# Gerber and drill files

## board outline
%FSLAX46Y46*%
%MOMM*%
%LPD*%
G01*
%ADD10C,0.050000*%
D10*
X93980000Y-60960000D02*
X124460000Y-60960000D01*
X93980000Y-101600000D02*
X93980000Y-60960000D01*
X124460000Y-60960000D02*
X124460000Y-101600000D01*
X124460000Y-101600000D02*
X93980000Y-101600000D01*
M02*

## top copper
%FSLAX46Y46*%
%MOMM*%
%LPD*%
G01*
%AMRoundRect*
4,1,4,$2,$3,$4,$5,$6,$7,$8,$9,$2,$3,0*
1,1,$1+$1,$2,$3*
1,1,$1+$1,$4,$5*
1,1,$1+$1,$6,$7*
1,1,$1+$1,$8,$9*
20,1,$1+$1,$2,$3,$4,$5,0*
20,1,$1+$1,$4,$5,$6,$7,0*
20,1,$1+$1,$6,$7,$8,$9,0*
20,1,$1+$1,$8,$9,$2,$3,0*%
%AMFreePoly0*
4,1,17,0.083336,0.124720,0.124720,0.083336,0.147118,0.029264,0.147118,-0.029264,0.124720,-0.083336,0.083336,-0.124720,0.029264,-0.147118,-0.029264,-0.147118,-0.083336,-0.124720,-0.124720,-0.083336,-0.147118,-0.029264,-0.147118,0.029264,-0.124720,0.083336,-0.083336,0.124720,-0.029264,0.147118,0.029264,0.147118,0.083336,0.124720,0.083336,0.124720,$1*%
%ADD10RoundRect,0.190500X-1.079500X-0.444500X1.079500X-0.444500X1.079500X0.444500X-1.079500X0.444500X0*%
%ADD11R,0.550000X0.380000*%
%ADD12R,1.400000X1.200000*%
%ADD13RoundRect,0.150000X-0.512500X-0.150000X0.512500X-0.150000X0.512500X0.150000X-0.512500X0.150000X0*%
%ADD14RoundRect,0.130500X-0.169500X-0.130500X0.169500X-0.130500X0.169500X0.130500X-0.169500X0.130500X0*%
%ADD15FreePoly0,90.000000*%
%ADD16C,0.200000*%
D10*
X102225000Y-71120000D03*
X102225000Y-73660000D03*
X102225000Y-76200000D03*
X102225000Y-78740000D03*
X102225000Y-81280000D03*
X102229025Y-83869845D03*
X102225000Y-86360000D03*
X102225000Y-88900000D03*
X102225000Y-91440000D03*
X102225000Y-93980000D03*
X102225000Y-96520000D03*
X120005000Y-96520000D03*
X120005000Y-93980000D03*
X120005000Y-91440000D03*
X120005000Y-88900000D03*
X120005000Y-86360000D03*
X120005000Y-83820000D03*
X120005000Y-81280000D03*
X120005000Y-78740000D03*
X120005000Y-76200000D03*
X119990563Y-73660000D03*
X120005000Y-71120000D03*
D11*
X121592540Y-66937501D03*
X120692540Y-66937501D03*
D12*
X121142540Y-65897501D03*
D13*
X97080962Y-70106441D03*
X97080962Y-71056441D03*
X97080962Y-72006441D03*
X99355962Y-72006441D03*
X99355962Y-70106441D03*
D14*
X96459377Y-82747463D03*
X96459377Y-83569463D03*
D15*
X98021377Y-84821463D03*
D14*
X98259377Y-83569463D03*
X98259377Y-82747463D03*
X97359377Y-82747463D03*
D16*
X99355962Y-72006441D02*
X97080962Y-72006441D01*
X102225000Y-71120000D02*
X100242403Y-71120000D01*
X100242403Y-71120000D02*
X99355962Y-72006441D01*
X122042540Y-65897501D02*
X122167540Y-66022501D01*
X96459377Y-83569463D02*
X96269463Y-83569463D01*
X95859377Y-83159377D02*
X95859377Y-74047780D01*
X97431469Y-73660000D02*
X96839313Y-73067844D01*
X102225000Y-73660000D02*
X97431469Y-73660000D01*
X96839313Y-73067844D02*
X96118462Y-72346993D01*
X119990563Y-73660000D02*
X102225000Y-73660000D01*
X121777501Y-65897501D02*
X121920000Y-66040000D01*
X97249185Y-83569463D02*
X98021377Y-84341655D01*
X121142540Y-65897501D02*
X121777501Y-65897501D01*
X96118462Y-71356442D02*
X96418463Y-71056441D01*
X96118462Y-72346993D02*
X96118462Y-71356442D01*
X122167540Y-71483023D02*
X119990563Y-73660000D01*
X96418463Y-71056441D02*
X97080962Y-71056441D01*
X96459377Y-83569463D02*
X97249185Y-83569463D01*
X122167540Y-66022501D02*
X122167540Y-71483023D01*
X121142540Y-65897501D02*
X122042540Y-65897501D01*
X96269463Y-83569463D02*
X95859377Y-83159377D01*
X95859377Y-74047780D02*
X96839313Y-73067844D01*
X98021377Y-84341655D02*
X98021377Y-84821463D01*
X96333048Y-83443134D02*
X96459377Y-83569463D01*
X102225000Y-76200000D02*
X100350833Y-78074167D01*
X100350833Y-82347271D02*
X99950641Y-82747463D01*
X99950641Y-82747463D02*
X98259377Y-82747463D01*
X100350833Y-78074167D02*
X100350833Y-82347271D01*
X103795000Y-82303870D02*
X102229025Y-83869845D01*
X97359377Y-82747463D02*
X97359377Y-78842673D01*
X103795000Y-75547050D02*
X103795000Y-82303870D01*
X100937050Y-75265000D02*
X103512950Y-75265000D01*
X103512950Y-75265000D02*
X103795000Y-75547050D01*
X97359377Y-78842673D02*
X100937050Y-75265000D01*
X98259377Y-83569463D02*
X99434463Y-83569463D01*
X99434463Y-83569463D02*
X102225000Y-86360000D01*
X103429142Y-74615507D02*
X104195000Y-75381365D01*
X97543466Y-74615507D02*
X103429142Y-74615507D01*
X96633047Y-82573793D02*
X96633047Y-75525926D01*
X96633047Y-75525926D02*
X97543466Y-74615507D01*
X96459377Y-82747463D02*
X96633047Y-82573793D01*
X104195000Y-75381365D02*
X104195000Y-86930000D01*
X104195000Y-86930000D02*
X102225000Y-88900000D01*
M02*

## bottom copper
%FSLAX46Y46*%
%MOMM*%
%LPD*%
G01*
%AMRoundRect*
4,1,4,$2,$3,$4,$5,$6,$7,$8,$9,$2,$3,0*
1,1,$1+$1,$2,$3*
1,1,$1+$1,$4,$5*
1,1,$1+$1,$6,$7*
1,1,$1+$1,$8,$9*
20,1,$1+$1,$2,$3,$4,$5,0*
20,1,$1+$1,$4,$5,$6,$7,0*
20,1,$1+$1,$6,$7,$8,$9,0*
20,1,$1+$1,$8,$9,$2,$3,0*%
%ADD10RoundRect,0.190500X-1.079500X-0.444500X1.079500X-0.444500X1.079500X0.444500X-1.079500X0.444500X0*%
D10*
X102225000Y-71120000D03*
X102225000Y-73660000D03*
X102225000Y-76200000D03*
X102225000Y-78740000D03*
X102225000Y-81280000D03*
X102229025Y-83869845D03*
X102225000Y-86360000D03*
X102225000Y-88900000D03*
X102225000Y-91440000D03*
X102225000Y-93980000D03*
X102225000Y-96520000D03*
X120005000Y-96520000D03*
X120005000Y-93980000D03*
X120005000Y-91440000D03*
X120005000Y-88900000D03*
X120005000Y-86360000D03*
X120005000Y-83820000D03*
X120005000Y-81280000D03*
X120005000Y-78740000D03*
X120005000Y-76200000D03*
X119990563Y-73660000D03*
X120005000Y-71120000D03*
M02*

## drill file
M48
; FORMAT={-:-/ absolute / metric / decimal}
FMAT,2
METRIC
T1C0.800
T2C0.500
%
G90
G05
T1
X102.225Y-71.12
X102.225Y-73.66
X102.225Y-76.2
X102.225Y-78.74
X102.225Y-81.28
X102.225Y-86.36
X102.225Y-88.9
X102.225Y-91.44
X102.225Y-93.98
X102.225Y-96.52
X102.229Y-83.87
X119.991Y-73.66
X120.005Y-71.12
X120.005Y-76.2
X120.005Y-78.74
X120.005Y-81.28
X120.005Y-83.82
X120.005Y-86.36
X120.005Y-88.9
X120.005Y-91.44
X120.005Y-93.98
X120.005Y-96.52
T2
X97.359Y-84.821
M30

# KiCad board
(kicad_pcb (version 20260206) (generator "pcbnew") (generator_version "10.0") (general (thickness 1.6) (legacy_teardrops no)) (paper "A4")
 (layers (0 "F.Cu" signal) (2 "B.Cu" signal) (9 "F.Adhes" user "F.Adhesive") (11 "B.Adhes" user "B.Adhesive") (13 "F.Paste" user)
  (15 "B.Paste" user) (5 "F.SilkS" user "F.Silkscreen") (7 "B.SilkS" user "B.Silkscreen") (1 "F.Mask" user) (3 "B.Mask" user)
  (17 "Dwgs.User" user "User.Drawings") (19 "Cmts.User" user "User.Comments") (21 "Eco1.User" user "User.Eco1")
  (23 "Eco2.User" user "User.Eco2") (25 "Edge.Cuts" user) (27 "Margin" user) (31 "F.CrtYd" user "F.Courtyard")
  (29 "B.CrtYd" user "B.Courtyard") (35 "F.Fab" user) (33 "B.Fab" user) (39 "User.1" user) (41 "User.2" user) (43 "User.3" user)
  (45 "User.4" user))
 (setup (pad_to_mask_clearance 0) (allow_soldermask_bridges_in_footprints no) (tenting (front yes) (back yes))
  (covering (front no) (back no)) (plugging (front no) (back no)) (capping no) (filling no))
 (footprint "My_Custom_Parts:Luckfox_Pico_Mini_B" (layer "F.Cu") (at 111.145 83.82)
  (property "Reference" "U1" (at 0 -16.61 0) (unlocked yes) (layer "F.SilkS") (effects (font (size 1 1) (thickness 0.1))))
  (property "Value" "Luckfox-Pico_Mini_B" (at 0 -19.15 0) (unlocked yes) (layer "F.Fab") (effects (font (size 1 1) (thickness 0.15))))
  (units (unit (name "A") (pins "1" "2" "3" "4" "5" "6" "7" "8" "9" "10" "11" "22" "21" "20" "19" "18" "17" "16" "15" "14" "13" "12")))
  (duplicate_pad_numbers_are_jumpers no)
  (pad "1" thru_hole roundrect (at -8.92 -12.7) (size 2.54 1.27) (drill 0.8) (layers "*.Cu" "*.Mask") (remove_unused_layers no)
   (roundrect_rratio 0.15) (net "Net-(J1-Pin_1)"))
  (pad "2" thru_hole roundrect (at -8.92 -10.16) (size 2.54 1.27) (drill 0.8) (layers "*.Cu" "*.Mask") (remove_unused_layers no)
   (roundrect_rratio 0.15) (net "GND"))
  (pad "3" thru_hole roundrect (at -8.92 -7.62) (size 2.54 1.27) (drill 0.8) (layers "*.Cu" "*.Mask") (remove_unused_layers no)
   (roundrect_rratio 0.15) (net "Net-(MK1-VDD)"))
  (pad "4" thru_hole roundrect (at -8.92 -5.08) (size 2.54 1.27) (drill 0.8) (layers "*.Cu" "*.Mask") (remove_unused_layers no)
   (roundrect_rratio 0.15) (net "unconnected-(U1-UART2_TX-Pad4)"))
  (pad "5" thru_hole roundrect (at -8.92 -2.54) (size 2.54 1.27) (drill 0.8) (layers "*.Cu" "*.Mask") (remove_unused_layers no)
   (roundrect_rratio 0.15) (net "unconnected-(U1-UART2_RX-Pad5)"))
  (pad "6" thru_hole roundrect (at -8.915975 0.049845) (size 2.54 1.27) (drill 0.8) (layers "*.Cu" "*.Mask") (remove_unused_layers no)
   (roundrect_rratio 0.15) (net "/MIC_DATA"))
  (pad "7" thru_hole roundrect (at -8.92 2.54) (size 2.54 1.27) (drill 0.8) (layers "*.Cu" "*.Mask") (remove_unused_layers no)
   (roundrect_rratio 0.15) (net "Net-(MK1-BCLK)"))
  (pad "8" thru_hole roundrect (at -8.92 5.08) (size 2.54 1.27) (drill 0.8) (layers "*.Cu" "*.Mask") (remove_unused_layers no)
   (roundrect_rratio 0.15) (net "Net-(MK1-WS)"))
  (pad "9" thru_hole roundrect (at -8.92 7.62) (size 2.54 1.27) (drill 0.8) (layers "*.Cu" "*.Mask") (remove_unused_layers no)
   (roundrect_rratio 0.15) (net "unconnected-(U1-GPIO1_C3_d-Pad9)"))
  (pad "10" thru_hole roundrect (at -8.92 10.16) (size 2.54 1.27) (drill 0.8) (layers "*.Cu" "*.Mask") (remove_unused_layers no)
   (roundrect_rratio 0.15) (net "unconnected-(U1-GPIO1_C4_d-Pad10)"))
  (pad "11" thru_hole roundrect (at -8.92 12.7) (size 2.54 1.27) (drill 0.8) (layers "*.Cu" "*.Mask") (remove_unused_layers no)
   (roundrect_rratio 0.15) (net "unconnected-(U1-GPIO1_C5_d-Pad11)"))
  (pad "12" thru_hole roundrect (at 8.86 12.7) (size 2.54 1.27) (drill 0.8) (layers "*.Cu" "*.Mask") (remove_unused_layers no)
   (roundrect_rratio 0.15) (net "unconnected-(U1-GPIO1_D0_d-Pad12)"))
  (pad "13" thru_hole roundrect (at 8.86 10.16) (size 2.54 1.27) (drill 0.8) (layers "*.Cu" "*.Mask") (remove_unused_layers no)
   (roundrect_rratio 0.15) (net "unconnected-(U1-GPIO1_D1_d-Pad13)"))
  (pad "14" thru_hole roundrect (at 8.86 7.62) (size 2.54 1.27) (drill 0.8) (layers "*.Cu" "*.Mask") (remove_unused_layers no)
   (roundrect_rratio 0.15) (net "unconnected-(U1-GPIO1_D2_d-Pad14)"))
  (pad "15" thru_hole roundrect (at 8.86 5.08) (size 2.54 1.27) (drill 0.8) (layers "*.Cu" "*.Mask") (remove_unused_layers no)
   (roundrect_rratio 0.15) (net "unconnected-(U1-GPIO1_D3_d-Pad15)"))
  (pad "16" thru_hole roundrect (at 8.86 2.54) (size 2.54 1.27) (drill 0.8) (layers "*.Cu" "*.Mask") (remove_unused_layers no)
   (roundrect_rratio 0.15) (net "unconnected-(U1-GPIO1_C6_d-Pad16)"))
  (pad "17" thru_hole roundrect (at 8.86 0) (size 2.54 1.27) (drill 0.8) (layers "*.Cu" "*.Mask") (remove_unused_layers no)
   (roundrect_rratio 0.15) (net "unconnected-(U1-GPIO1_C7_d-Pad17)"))
  (pad "18" thru_hole roundrect (at 8.86 -2.54) (size 2.54 1.27) (drill 0.8) (layers "*.Cu" "*.Mask") (remove_unused_layers no)
   (roundrect_rratio 0.15) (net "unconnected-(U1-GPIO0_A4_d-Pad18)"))
  (pad "19" thru_hole roundrect (at 8.86 -5.08) (size 2.54 1.27) (drill 0.8) (layers "*.Cu" "*.Mask") (remove_unused_layers no)
   (roundrect_rratio 0.15) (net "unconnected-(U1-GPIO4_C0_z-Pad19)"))
  (pad "20" thru_hole roundrect (at 8.86 -7.62) (size 2.54 1.27) (drill 0.8) (layers "*.Cu" "*.Mask") (remove_unused_layers no)
   (roundrect_rratio 0.15) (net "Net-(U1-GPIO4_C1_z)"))
  (pad "21" thru_hole roundrect (at 8.845563 -10.16) (size 2.54 1.27) (drill 0.8) (layers "*.Cu" "*.Mask") (remove_unused_layers no)
   (roundrect_rratio 0.15) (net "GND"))
  (pad "22" thru_hole roundrect (at 8.86 -12.7) (size 2.54 1.27) (drill 0.8) (layers "*.Cu" "*.Mask") (remove_unused_layers no)
   (roundrect_rratio 0.15) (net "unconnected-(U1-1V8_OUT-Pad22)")))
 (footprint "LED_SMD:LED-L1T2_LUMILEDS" (layer "F.Cu") (at 121.14254 66.417501)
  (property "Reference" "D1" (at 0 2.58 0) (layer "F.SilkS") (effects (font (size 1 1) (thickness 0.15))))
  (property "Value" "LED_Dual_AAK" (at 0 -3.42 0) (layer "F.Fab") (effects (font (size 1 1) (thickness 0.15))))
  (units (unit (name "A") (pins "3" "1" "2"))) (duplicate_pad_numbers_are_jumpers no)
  (pad "1" smd rect (at 0.45 0.52) (size 0.55 0.38) (layers "F.Cu" "F.Mask" "F.Paste") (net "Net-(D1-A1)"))
  (pad "2" smd rect (at -0.45 0.52) (size 0.55 0.38) (layers "F.Cu" "F.Mask" "F.Paste") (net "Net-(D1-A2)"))
  (pad "3" smd rect (at 0 -0.52) (size 1.4 1.2) (layers "F.Cu" "F.Mask" "F.Paste") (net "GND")))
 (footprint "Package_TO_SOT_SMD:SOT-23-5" (layer "F.Cu") (at 98.218462 71.056441)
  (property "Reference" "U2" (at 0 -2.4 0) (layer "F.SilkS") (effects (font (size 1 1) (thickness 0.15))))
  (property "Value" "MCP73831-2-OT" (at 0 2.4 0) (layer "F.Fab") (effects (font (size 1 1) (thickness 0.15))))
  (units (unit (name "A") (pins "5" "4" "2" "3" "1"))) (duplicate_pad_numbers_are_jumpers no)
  (pad "1" smd roundrect (at -1.1375 -0.95) (size 1.325 0.6) (layers "F.Cu" "F.Mask" "F.Paste") (roundrect_rratio 0.25)
   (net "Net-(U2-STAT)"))
  (pad "2" smd roundrect (at -1.1375 0) (size 1.325 0.6) (layers "F.Cu" "F.Mask" "F.Paste") (roundrect_rratio 0.25) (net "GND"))
  (pad "3" smd roundrect (at -1.1375 0.95) (size 1.325 0.6) (layers "F.Cu" "F.Mask" "F.Paste") (roundrect_rratio 0.25)
   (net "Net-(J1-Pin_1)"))
  (pad "4" smd roundrect (at 1.1375 0.95) (size 1.325 0.6) (layers "F.Cu" "F.Mask" "F.Paste") (roundrect_rratio 0.25) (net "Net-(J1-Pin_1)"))
  (pad "5" smd roundrect (at 1.1375 -0.95) (size 1.325 0.6) (layers "F.Cu" "F.Mask" "F.Paste") (roundrect_rratio 0.25) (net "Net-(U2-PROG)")))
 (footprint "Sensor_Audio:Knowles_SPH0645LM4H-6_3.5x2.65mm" (layer "F.Cu") (at 97.359377 84.111463)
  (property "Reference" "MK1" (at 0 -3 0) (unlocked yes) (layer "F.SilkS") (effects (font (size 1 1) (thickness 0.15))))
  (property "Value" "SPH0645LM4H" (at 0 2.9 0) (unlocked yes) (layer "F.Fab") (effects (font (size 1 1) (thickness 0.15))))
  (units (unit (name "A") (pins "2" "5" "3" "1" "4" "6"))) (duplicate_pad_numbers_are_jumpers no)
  (pad "" np_thru_hole circle (at 0 0.71) (size 0.5 0.5) (drill 0.5) (layers "*.Mask"))
  (pad "1" smd roundrect (at -0.9 -1.364) (size 0.6 0.522) (layers "F.Cu" "F.Mask" "F.Paste") (roundrect_rratio 0.25) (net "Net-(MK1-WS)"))
  (pad "2" smd roundrect (at -0.9 -0.542) (size 0.6 0.522) (layers "F.Cu" "F.Mask" "F.Paste") (roundrect_rratio 0.25) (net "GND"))
  (pad "3" smd custom (at 0.662 0.71 90) (size 0.3 0.3) (layers "F.Cu" "F.Mask") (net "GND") (options (clearance outline) (anchor circle))
   (primitives))
  (pad "4" smd roundrect (at 0.9 -0.542) (size 0.6 0.522) (layers "F.Cu" "F.Mask" "F.Paste") (roundrect_rratio 0.25) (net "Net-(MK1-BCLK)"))
  (pad "5" smd roundrect (at 0.9 -1.364) (size 0.6 0.522) (layers "F.Cu" "F.Mask" "F.Paste") (roundrect_rratio 0.25) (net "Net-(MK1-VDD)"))
  (pad "6" smd roundrect (at 0 -1.364) (size 0.6 0.522) (layers "F.Cu" "F.Mask" "F.Paste") (roundrect_rratio 0.25) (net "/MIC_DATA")))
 (gr_line (start 93.98 60.96) (end 124.46 60.96) (stroke (width 0.05) (type default)) (layer "Edge.Cuts"))
 (gr_line (start 93.98 101.6) (end 93.98 60.96) (stroke (width 0.05) (type default)) (layer "Edge.Cuts"))
 (gr_line (start 124.46 60.96) (end 124.46 101.6) (stroke (width 0.05) (type default)) (layer "Edge.Cuts"))
 (gr_line (start 124.46 101.6) (end 93.98 101.6) (stroke (width 0.05) (type default)) (layer "Edge.Cuts"))
 (segment (start 99.355962 72.006441) (end 97.080962 72.006441) (width 0.2) (layer "F.Cu") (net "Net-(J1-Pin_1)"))
 (segment (start 102.225 71.12) (end 100.242403 71.12) (width 0.2) (layer "F.Cu") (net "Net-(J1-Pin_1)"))
 (segment (start 100.242403 71.12) (end 99.355962 72.006441) (width 0.2) (layer "F.Cu") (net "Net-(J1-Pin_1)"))
 (segment (start 122.04254 65.897501) (end 122.16754 66.022501) (width 0.2) (layer "F.Cu") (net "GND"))
 (segment (start 96.459377 83.569463) (end 96.269463 83.569463) (width 0.2) (layer "F.Cu") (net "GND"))
 (segment (start 95.859377 83.159377) (end 95.859377 74.04778) (width 0.2) (layer "F.Cu") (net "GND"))
 (segment (start 97.431469 73.66) (end 96.839313 73.067844) (width 0.2) (layer "F.Cu") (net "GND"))
 (segment (start 102.225 73.66) (end 97.431469 73.66) (width 0.2) (layer "F.Cu") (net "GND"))
 (segment (start 96.839313 73.067844) (end 96.118462 72.346993) (width 0.2) (layer "F.Cu") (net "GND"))
 (segment (start 119.990563 73.66) (end 102.225 73.66) (width 0.2) (layer "F.Cu") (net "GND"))
 (segment (start 121.777501 65.897501) (end 121.92 66.04) (width 0.2) (layer "F.Cu") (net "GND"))
 (segment (start 97.249185 83.569463) (end 98.021377 84.341655) (width 0.2) (layer "F.Cu") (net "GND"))
 (segment (start 121.14254 65.897501) (end 121.777501 65.897501) (width 0.2) (layer "F.Cu") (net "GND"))
 (segment (start 96.118462 71.356442) (end 96.418463 71.056441) (width 0.2) (layer "F.Cu") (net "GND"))
 (segment (start 96.118462 72.346993) (end 96.118462 71.356442) (width 0.2) (layer "F.Cu") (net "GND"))
 (segment (start 122.16754 71.483023) (end 119.990563 73.66) (width 0.2) (layer "F.Cu") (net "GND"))
 (segment (start 96.418463 71.056441) (end 97.080962 71.056441) (width 0.2) (layer "F.Cu") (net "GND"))
 (segment (start 96.459377 83.569463) (end 97.249185 83.569463) (width 0.2) (layer "F.Cu") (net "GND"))
 (segment (start 122.16754 66.022501) (end 122.16754 71.483023) (width 0.2) (layer "F.Cu") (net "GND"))
 (segment (start 121.14254 65.897501) (end 122.04254 65.897501) (width 0.2) (layer "F.Cu") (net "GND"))
 (segment (start 96.269463 83.569463) (end 95.859377 83.159377) (width 0.2) (layer "F.Cu") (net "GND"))
 (segment (start 95.859377 74.04778) (end 96.839313 73.067844) (width 0.2) (layer "F.Cu") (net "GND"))
 (segment (start 98.021377 84.341655) (end 98.021377 84.821463) (width 0.2) (layer "F.Cu") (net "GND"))
 (segment (start 96.333048 83.443134) (end 96.459377 83.569463) (width 0.2) (layer "F.Cu") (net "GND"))
 (segment (start 102.225 76.2) (end 100.350833 78.074167) (width 0.2) (layer "F.Cu") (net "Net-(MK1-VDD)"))
 (segment (start 100.350833 82.347271) (end 99.950641 82.747463) (width 0.2) (layer "F.Cu") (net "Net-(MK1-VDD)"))
 (segment (start 99.950641 82.747463) (end 98.259377 82.747463) (width 0.2) (layer "F.Cu") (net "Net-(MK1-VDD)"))
 (segment (start 100.350833 78.074167) (end 100.350833 82.347271) (width 0.2) (layer "F.Cu") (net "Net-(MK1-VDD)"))
 (segment (start 103.795 82.30387) (end 102.229025 83.869845) (width 0.2) (layer "F.Cu") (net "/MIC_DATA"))
 (segment (start 97.359377 82.747463) (end 97.359377 78.842673) (width 0.2) (layer "F.Cu") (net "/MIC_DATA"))
 (segment (start 103.795 75.54705) (end 103.795 82.30387) (width 0.2) (layer "F.Cu") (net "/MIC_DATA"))
 (segment (start 100.93705 75.265) (end 103.51295 75.265) (width 0.2) (layer "F.Cu") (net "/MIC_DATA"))
 (segment (start 103.51295 75.265) (end 103.795 75.54705) (width 0.2) (layer "F.Cu") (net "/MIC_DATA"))
 (segment (start 97.359377 78.842673) (end 100.93705 75.265) (width 0.2) (layer "F.Cu") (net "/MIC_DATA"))
 (segment (start 98.259377 83.569463) (end 99.434463 83.569463) (width 0.2) (layer "F.Cu") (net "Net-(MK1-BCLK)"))
 (segment (start 99.434463 83.569463) (end 102.225 86.36) (width 0.2) (layer "F.Cu") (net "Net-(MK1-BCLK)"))
 (segment (start 103.429142 74.615507) (end 104.195 75.381365) (width 0.2) (layer "F.Cu") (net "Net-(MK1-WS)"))
 (segment (start 97.543466 74.615507) (end 103.429142 74.615507) (width 0.2) (layer "F.Cu") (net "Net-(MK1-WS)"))
 (segment (start 96.633047 82.573793) (end 96.633047 75.525926) (width 0.2) (layer "F.Cu") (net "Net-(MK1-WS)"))
 (segment (start 96.633047 75.525926) (end 97.543466 74.615507) (width 0.2) (layer "F.Cu") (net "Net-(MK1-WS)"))
 (segment (start 96.459377 82.747463) (end 96.633047 82.573793) (width 0.2) (layer "F.Cu") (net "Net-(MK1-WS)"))
 (segment (start 104.195 75.381365) (end 104.195 86.93) (width 0.2) (layer "F.Cu") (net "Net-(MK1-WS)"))
 (segment (start 104.195 86.93) (end 102.225 88.9) (width 0.2) (layer "F.Cu") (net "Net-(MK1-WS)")))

